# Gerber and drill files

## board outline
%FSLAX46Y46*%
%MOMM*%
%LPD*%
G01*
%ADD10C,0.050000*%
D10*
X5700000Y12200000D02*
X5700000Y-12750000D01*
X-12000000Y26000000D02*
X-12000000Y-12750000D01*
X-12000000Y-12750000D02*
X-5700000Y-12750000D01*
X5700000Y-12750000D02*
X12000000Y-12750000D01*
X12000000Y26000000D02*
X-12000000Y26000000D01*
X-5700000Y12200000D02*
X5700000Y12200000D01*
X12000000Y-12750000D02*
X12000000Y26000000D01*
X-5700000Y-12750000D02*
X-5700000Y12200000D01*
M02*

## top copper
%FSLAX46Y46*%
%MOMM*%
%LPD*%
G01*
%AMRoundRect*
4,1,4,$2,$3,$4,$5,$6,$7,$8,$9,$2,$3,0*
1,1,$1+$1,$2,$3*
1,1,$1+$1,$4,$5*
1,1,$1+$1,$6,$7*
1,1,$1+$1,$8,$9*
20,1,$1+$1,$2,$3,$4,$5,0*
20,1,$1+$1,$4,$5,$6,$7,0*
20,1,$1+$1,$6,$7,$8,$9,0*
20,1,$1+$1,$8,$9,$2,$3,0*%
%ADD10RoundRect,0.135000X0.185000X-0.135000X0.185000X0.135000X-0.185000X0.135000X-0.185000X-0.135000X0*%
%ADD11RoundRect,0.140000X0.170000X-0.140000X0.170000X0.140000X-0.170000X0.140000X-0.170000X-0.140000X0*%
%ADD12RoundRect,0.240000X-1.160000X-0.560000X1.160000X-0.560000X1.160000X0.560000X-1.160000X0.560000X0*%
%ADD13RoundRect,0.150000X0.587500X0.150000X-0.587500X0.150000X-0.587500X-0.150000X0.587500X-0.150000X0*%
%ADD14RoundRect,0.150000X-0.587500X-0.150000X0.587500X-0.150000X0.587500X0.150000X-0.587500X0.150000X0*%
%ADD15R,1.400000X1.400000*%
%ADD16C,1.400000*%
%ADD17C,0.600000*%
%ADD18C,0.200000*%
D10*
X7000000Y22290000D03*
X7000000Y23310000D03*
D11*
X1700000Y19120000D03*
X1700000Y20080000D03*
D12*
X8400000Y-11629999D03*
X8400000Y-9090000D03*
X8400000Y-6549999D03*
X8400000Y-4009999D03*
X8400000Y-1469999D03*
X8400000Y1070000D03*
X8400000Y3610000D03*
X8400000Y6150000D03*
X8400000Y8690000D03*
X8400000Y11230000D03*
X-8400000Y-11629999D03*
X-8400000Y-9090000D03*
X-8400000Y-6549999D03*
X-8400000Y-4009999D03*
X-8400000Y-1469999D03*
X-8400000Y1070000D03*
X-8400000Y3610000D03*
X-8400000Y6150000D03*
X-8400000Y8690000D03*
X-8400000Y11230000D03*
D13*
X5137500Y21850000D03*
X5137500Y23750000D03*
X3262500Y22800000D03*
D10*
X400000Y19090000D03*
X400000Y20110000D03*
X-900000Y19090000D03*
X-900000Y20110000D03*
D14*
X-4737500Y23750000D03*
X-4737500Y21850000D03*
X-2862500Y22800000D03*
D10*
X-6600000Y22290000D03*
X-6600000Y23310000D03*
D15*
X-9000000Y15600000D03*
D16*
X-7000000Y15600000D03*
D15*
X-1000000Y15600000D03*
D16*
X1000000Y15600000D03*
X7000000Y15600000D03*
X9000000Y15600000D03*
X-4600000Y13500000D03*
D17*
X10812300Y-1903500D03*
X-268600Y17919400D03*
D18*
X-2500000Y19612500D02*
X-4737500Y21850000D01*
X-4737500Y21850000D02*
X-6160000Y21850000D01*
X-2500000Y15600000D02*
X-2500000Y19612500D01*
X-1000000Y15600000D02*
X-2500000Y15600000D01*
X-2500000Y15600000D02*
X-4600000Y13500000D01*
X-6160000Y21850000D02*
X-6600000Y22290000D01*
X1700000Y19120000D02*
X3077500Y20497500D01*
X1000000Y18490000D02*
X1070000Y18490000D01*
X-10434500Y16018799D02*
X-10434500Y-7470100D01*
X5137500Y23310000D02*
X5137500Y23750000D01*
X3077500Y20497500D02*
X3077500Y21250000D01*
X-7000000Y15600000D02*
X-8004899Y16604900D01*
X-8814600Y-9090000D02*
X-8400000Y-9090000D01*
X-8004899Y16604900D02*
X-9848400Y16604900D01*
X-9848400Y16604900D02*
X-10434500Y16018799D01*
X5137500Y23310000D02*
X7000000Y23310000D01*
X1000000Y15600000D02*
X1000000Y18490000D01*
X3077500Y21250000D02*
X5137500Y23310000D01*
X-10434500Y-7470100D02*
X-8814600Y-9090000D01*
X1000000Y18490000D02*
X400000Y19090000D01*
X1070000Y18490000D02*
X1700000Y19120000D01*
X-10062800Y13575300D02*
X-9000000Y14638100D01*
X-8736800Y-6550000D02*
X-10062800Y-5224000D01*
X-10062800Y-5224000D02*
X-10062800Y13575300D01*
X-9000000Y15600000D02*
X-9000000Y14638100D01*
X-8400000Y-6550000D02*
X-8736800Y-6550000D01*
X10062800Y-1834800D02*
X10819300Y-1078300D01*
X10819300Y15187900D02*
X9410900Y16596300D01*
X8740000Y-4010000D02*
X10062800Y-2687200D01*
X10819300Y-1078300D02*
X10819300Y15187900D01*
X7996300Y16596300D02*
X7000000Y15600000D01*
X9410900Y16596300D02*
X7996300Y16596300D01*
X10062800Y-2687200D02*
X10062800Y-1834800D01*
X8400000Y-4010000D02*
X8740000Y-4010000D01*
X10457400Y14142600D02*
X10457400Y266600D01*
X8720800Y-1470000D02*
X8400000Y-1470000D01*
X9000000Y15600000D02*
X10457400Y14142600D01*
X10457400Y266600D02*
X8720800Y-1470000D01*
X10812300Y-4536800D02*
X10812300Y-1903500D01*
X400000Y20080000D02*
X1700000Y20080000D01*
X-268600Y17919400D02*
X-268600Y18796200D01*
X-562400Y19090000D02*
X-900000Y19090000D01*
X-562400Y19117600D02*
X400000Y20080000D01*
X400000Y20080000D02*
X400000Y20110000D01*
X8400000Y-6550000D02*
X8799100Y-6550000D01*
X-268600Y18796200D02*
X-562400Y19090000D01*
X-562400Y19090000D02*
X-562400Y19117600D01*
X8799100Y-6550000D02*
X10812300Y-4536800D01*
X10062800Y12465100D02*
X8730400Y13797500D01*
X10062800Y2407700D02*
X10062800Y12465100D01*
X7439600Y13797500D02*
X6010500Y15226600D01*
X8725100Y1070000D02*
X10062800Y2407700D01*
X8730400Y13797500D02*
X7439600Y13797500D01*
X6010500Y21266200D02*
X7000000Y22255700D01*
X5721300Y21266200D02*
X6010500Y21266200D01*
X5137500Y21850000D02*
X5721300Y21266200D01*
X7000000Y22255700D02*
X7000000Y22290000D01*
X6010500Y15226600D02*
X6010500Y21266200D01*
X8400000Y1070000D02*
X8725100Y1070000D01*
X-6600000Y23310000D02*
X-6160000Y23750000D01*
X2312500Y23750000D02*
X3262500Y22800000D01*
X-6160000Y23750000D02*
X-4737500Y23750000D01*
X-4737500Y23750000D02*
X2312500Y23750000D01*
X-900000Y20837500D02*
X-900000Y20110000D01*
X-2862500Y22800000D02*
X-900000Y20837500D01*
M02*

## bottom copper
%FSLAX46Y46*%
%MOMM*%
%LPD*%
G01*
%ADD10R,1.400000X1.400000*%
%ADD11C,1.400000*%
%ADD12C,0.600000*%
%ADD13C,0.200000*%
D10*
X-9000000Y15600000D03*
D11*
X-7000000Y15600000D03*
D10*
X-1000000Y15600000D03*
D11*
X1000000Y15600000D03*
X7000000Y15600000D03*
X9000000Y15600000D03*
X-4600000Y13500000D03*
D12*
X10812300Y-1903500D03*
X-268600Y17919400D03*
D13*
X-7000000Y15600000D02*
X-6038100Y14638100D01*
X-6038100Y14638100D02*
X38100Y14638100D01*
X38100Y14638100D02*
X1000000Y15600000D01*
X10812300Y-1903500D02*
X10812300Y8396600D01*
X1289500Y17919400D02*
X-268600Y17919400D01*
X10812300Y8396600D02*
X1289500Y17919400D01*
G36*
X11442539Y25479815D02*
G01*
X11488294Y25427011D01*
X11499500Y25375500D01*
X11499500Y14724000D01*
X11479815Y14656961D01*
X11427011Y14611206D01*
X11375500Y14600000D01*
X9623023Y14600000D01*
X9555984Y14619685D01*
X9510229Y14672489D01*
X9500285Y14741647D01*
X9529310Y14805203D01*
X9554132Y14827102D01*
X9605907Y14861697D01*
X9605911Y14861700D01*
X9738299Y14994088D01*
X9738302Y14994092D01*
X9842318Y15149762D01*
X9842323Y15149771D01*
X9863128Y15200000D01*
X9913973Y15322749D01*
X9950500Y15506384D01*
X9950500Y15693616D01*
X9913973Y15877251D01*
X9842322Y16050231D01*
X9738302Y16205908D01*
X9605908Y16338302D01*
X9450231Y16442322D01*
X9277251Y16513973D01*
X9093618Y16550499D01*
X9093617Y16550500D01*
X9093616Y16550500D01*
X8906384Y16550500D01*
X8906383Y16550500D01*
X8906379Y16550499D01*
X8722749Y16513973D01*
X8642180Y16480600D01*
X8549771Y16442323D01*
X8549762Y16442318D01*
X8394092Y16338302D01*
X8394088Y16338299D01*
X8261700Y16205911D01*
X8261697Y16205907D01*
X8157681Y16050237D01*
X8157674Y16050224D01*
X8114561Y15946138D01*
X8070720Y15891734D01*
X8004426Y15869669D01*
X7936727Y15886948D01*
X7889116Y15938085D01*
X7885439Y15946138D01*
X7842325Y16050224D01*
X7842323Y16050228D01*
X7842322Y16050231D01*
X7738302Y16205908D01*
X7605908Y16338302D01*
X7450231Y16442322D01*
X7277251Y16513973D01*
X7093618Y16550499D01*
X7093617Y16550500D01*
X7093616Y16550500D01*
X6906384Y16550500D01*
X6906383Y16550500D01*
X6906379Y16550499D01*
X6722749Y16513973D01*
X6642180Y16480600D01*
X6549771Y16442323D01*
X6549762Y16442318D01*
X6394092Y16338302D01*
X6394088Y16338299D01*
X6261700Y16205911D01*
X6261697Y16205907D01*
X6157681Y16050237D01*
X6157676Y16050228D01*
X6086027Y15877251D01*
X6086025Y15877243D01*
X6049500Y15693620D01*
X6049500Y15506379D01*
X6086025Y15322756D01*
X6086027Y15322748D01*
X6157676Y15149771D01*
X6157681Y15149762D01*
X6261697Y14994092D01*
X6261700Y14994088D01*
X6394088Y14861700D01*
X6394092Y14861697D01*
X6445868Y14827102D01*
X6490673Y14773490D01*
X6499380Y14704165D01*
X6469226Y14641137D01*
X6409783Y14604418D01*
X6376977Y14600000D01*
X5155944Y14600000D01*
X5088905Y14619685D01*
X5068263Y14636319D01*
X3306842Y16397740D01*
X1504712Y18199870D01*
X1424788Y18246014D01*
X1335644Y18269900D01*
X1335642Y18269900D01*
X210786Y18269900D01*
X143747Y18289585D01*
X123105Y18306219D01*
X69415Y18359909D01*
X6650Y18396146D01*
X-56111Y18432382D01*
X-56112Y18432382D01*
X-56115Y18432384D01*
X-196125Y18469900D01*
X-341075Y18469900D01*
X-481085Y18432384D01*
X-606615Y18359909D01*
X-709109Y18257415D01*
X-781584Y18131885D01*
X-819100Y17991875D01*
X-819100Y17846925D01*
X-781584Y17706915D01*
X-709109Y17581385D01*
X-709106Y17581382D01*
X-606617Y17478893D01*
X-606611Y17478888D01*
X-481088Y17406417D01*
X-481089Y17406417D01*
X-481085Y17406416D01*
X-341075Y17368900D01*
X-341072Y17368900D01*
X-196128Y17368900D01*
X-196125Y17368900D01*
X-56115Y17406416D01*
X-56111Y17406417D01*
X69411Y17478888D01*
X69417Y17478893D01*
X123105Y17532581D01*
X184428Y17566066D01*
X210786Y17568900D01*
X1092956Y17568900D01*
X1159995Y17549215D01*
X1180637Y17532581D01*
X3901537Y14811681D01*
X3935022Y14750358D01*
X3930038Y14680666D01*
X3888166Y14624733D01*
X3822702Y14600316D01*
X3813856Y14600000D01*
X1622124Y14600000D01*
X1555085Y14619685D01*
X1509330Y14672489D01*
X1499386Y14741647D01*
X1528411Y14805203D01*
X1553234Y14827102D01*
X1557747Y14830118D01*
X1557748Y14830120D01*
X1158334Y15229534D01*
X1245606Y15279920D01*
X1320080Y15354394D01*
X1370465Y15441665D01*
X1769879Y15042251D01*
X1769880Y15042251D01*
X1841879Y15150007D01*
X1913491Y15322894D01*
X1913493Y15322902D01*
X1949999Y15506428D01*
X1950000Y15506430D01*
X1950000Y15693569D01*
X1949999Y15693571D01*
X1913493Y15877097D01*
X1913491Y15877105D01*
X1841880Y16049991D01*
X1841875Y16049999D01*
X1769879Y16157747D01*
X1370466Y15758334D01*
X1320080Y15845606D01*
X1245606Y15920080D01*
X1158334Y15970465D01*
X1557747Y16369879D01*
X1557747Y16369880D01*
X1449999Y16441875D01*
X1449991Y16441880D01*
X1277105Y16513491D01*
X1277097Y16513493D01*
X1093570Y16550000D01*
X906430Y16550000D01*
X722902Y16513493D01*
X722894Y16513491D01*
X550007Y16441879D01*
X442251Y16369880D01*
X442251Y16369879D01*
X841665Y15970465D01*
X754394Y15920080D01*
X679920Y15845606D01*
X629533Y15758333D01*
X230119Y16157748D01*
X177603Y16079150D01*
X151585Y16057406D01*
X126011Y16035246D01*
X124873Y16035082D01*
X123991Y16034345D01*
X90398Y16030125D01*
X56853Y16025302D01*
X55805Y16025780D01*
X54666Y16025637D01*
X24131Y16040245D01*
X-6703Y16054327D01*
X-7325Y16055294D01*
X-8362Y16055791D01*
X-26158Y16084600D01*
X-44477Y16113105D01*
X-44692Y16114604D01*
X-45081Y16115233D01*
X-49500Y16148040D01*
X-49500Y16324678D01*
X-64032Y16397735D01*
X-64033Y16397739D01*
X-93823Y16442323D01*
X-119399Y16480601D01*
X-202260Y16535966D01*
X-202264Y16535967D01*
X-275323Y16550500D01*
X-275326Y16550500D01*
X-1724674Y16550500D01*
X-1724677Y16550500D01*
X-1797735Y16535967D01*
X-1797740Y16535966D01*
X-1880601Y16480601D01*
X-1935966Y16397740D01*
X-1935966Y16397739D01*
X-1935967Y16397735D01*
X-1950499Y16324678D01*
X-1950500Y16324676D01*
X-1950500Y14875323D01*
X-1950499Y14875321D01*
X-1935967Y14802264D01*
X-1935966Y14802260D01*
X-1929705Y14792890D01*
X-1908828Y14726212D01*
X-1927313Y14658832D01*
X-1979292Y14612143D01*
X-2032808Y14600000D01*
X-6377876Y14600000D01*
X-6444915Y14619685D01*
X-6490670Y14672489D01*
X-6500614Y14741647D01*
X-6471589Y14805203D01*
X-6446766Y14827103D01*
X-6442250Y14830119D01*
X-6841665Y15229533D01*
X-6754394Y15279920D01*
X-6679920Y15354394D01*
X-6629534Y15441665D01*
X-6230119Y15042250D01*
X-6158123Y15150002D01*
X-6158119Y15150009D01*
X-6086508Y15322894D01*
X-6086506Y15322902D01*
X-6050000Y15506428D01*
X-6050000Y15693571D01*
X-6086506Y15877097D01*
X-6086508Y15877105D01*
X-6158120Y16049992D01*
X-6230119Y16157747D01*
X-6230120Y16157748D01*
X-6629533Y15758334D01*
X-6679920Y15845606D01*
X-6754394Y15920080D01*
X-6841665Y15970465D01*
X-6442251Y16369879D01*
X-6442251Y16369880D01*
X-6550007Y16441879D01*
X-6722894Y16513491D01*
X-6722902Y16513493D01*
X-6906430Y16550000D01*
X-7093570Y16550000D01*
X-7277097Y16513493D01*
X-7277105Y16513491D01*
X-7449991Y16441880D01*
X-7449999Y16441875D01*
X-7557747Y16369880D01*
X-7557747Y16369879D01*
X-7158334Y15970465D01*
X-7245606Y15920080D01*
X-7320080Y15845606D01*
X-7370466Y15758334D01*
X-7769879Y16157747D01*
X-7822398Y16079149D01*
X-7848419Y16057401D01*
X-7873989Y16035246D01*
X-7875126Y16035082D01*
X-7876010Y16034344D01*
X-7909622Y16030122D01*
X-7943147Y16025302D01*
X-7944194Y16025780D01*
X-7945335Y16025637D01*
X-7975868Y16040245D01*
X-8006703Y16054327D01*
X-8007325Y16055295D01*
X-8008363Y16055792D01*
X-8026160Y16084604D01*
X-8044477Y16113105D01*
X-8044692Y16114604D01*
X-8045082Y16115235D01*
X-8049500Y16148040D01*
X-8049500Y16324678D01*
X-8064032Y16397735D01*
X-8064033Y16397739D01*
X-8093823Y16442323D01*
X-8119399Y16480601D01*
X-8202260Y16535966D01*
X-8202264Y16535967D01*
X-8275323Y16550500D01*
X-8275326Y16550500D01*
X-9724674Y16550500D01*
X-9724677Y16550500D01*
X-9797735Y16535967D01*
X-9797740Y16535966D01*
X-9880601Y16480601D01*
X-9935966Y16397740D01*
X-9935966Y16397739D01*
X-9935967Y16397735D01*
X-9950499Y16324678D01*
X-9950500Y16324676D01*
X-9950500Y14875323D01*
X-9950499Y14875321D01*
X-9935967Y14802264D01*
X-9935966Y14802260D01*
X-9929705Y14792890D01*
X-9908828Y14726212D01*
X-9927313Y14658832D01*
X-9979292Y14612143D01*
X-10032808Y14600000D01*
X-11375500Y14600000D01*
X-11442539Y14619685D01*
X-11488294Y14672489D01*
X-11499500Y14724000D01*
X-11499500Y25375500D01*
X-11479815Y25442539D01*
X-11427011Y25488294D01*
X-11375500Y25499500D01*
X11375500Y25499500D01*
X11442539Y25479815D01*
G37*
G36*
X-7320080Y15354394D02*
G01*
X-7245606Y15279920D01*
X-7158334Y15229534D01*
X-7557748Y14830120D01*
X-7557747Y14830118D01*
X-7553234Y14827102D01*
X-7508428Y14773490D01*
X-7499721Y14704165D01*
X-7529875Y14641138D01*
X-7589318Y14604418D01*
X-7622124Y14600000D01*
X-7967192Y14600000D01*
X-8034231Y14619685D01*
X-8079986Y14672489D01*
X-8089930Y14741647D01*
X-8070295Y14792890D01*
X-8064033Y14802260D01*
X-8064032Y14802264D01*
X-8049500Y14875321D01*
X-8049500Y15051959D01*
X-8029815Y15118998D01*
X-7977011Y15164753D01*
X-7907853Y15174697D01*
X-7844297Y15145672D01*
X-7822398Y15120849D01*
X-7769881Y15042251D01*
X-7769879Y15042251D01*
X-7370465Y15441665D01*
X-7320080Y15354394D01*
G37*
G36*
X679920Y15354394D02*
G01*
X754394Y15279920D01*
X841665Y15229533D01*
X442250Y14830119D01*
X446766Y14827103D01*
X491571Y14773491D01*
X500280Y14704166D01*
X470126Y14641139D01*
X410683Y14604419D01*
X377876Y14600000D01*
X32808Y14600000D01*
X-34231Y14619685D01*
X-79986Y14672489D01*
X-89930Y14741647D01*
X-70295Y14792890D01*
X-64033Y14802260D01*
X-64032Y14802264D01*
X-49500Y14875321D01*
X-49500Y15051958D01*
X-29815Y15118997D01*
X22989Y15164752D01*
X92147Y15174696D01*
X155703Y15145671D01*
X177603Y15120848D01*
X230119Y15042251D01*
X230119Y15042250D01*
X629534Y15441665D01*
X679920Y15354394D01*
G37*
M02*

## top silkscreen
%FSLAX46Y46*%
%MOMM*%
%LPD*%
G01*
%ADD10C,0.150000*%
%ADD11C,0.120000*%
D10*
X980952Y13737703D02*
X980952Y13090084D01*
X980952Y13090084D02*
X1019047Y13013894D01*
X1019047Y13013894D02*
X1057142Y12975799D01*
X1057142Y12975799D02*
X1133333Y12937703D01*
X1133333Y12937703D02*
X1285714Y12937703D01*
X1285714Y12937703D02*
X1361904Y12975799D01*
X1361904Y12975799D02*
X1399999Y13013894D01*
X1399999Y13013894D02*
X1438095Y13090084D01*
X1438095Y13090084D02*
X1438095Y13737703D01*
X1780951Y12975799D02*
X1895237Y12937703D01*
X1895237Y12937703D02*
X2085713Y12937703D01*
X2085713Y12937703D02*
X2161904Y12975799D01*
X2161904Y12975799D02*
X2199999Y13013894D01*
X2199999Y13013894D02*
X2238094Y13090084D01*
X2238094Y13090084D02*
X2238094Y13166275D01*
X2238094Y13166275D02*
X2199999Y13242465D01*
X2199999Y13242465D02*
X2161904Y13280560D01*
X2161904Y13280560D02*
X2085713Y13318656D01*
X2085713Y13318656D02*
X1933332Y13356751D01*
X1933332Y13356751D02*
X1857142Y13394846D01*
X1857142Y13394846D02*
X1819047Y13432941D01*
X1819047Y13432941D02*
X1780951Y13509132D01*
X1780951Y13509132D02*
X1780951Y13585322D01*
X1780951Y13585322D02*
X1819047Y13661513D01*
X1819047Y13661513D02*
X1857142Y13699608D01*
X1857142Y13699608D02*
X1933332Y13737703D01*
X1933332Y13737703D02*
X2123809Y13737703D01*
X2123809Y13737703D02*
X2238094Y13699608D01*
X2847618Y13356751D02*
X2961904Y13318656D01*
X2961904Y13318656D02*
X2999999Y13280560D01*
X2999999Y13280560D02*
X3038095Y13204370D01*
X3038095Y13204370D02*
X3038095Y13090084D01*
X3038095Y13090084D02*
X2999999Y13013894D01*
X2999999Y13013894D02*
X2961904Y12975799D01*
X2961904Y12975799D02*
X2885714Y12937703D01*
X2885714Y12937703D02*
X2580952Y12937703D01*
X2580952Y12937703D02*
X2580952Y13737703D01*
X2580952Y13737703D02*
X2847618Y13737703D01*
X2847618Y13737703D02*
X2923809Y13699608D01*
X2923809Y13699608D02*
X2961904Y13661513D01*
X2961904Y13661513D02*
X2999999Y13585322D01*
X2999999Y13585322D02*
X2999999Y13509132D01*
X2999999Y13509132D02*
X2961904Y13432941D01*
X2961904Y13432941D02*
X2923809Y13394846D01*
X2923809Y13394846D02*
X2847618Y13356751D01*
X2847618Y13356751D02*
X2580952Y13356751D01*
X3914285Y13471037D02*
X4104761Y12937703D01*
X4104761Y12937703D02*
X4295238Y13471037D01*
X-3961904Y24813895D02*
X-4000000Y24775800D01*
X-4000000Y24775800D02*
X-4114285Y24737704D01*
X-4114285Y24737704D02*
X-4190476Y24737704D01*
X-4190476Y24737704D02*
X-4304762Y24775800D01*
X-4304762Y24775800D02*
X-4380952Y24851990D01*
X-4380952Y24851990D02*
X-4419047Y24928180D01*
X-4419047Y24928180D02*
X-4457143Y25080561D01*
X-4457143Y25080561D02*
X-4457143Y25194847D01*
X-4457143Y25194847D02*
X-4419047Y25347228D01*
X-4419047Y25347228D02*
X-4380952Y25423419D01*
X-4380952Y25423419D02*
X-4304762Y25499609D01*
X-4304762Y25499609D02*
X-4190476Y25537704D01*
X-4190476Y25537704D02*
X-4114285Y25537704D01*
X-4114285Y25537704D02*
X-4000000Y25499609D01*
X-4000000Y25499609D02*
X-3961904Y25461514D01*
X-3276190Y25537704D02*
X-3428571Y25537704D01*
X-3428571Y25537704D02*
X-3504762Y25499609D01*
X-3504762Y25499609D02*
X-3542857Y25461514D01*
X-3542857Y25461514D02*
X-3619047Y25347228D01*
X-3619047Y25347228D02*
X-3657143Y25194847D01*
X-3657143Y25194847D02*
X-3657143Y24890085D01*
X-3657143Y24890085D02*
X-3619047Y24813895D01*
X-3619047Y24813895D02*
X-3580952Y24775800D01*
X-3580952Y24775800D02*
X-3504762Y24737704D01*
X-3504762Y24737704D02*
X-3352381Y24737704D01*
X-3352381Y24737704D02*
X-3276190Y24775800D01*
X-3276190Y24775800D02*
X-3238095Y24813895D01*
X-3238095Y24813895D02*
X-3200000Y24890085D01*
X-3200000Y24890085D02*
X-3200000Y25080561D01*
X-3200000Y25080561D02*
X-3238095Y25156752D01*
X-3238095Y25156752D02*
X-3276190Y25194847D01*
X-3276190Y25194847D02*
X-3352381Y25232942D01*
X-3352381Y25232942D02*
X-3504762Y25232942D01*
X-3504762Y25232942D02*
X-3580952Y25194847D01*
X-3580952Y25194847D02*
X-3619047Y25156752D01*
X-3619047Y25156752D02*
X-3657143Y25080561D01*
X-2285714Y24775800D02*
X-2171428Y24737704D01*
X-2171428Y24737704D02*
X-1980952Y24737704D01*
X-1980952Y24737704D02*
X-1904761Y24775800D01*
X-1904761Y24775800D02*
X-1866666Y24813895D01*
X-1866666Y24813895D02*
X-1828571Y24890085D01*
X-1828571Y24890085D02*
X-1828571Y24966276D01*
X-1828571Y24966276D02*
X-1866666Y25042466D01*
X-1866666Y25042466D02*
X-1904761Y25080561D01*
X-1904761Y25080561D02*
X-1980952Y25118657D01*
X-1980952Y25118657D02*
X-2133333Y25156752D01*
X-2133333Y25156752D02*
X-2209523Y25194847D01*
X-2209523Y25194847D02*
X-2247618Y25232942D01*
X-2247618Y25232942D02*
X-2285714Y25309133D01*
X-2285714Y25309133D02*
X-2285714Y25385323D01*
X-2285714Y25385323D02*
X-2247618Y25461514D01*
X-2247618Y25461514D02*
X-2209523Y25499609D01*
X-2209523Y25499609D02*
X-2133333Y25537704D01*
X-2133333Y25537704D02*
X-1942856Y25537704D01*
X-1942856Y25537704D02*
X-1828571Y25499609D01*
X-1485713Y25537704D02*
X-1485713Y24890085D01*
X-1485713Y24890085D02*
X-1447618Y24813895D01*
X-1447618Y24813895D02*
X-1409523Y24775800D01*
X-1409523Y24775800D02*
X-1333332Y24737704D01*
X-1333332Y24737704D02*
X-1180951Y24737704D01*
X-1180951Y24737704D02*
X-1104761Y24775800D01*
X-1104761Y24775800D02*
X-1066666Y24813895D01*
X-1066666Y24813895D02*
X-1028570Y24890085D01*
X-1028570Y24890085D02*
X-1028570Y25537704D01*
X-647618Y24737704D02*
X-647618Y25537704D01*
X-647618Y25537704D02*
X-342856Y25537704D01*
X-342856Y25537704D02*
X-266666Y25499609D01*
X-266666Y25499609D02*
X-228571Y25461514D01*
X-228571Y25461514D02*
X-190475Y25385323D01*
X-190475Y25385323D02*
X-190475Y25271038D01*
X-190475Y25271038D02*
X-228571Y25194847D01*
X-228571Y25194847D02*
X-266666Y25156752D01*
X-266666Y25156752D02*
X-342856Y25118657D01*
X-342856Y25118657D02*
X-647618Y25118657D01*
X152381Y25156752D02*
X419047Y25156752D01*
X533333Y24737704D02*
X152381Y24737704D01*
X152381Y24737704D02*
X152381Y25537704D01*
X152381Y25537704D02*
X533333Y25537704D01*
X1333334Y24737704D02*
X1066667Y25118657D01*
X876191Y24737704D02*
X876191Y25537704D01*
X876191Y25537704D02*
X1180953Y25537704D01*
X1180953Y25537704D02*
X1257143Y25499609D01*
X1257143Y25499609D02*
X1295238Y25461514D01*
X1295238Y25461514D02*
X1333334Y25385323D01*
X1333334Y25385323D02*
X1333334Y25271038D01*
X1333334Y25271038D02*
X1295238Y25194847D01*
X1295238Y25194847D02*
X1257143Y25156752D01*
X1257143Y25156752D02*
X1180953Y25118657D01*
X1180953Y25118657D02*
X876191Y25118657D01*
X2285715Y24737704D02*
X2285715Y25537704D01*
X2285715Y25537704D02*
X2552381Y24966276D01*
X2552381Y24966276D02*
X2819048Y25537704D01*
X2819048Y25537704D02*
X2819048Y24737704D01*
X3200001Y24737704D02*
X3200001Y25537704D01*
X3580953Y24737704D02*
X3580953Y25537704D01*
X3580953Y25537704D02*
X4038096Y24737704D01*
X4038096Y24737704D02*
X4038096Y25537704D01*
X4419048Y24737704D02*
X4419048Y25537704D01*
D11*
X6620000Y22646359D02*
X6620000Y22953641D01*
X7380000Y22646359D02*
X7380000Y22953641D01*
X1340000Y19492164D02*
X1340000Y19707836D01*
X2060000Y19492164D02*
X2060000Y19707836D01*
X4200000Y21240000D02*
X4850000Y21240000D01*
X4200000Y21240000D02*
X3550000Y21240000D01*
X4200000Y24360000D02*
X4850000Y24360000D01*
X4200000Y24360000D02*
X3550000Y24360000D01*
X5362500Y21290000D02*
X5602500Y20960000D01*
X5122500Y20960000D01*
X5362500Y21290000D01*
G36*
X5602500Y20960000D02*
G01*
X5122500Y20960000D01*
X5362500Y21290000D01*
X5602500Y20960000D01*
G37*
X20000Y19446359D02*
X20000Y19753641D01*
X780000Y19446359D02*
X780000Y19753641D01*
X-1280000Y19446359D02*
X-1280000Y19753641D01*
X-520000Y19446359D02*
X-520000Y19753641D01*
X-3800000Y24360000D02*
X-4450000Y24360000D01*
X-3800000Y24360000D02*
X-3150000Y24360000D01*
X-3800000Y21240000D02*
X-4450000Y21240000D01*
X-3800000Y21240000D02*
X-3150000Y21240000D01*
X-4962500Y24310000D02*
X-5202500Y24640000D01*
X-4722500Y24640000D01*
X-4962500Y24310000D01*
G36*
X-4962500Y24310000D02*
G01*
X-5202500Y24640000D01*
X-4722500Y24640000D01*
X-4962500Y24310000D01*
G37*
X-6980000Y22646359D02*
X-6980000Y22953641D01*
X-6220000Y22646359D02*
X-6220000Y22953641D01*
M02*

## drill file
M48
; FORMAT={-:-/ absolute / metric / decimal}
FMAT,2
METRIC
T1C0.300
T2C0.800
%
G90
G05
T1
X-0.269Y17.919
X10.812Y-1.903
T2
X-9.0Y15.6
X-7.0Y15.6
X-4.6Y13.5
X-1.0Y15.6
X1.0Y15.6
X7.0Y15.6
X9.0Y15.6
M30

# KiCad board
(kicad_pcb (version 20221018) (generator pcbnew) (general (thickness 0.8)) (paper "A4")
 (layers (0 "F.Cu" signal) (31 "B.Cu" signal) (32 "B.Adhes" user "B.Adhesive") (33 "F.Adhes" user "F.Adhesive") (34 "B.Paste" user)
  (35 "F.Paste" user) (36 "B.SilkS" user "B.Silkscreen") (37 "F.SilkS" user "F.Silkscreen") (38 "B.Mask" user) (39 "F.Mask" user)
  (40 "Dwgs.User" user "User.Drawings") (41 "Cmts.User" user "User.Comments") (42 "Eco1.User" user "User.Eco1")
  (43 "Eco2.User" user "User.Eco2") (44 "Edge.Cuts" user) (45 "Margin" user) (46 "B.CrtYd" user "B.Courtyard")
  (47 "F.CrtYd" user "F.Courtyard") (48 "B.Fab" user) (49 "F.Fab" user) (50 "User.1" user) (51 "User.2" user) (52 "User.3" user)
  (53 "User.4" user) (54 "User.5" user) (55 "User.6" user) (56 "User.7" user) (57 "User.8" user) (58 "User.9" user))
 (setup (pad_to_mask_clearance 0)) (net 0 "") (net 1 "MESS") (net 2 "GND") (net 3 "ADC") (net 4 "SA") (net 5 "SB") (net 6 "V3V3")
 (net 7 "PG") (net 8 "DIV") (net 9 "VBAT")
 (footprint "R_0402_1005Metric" (layer "F.Cu") (at 7 -22.8 90)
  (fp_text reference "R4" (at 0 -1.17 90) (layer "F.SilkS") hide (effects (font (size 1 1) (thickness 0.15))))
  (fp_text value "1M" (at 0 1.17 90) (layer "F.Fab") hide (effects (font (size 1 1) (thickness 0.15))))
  (fp_line (start -0.153641 -0.38) (end 0.153641 -0.38) (stroke (width 0.12) (type solid)) (layer "F.SilkS"))
  (fp_line (start -0.153641 0.38) (end 0.153641 0.38) (stroke (width 0.12) (type solid)) (layer "F.SilkS"))
  (pad "1" smd roundrect (at -0.51 0 90) (size 0.54 0.64) (layers "F.Cu" "F.Paste" "F.Mask") (roundrect_rratio 0.25) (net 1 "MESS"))
  (pad "2" smd roundrect (at 0.51 0 90) (size 0.54 0.64) (layers "F.Cu" "F.Paste" "F.Mask") (roundrect_rratio 0.25) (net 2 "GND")))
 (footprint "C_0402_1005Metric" (layer "F.Cu") (at 1.7 -19.6 90)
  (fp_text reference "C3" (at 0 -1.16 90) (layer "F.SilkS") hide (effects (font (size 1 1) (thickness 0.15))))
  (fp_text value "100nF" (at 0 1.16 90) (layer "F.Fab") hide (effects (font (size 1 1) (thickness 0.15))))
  (fp_line (start -0.107836 -0.36) (end 0.107836 -0.36) (stroke (width 0.12) (type solid)) (layer "F.SilkS"))
  (fp_line (start -0.107836 0.36) (end 0.107836 0.36) (stroke (width 0.12) (type solid)) (layer "F.SilkS"))
  (pad "1" smd roundrect (at -0.48 0 90) (size 0.56 0.62) (layers "F.Cu" "F.Paste" "F.Mask") (roundrect_rratio 0.25) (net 2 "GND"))
  (pad "2" smd roundrect (at 0.48 0 90) (size 0.56 0.62) (layers "F.Cu" "F.Paste" "F.Mask") (roundrect_rratio 0.25) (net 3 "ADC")))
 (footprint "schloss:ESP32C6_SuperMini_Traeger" (layer "F.Cu") (at 0 0)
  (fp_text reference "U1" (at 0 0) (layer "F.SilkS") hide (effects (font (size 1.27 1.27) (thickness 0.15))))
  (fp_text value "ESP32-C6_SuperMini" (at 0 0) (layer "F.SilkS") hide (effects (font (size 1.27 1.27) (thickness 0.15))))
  (pad "1" smd roundrect (at 8.4 11.629999) (size 2.8 1.6) (layers "F.Cu" "F.Mask") (roundrect_rratio 0.15) (thermal_bridge_angle 45))
  (pad "2" smd roundrect (at 8.4 9.09) (size 2.8 1.6) (layers "F.Cu" "F.Mask") (roundrect_rratio 0.15) (thermal_bridge_angle 45))
  (pad "3" smd roundrect (at 8.4 6.549999) (size 2.8 1.6) (layers "F.Cu" "F.Mask") (roundrect_rratio 0.15) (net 3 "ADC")
   (thermal_bridge_angle 45))
  (pad "4" smd roundrect (at 8.4 4.009999) (size 2.8 1.6) (layers "F.Cu" "F.Mask") (roundrect_rratio 0.15) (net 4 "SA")
   (thermal_bridge_angle 45))
  (pad "5" smd roundrect (at 8.4 1.469999) (size 2.8 1.6) (layers "F.Cu" "F.Mask") (roundrect_rratio 0.15) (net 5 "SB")
   (thermal_bridge_angle 45))
  (pad "6" smd roundrect (at 8.4 -1.07) (size 2.8 1.6) (layers "F.Cu" "F.Mask") (roundrect_rratio 0.15) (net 1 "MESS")
   (thermal_bridge_angle 45))
  (pad "7" smd roundrect (at 8.4 -3.61) (size 2.8 1.6) (layers "F.Cu" "F.Mask") (roundrect_rratio 0.15) (thermal_bridge_angle 45))
  (pad "8" smd roundrect (at 8.4 -6.15) (size 2.8 1.6) (layers "F.Cu" "F.Mask") (roundrect_rratio 0.15) (thermal_bridge_angle 45))
  (pad "9" smd roundrect (at 8.4 -8.69) (size 2.8 1.6) (layers "F.Cu" "F.Mask") (roundrect_rratio 0.15) (thermal_bridge_angle 45))
  (pad "10" smd roundrect (at 8.4 -11.23) (size 2.8 1.6) (layers "F.Cu" "F.Mask") (roundrect_rratio 0.15) (thermal_bridge_angle 45))
  (pad "11" smd roundrect (at -8.4 11.629999) (size 2.8 1.6) (layers "F.Cu" "F.Mask") (roundrect_rratio 0.15) (thermal_bridge_angle 45))
  (pad "12" smd roundrect (at -8.4 9.09) (size 2.8 1.6) (layers "F.Cu" "F.Mask") (roundrect_rratio 0.15) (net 2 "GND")
   (thermal_bridge_angle 45))
  (pad "13" smd roundrect (at -8.4 6.549999) (size 2.8 1.6) (layers "F.Cu" "F.Mask") (roundrect_rratio 0.15) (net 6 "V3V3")
   (thermal_bridge_angle 45))
  (pad "14" smd roundrect (at -8.4 4.009999) (size 2.8 1.6) (layers "F.Cu" "F.Mask") (roundrect_rratio 0.15) (thermal_bridge_angle 45))
  (pad "15" smd roundrect (at -8.4 1.469999) (size 2.8 1.6) (layers "F.Cu" "F.Mask") (roundrect_rratio 0.15) (thermal_bridge_angle 45))
  (pad "16" smd roundrect (at -8.4 -1.07) (size 2.8 1.6) (layers "F.Cu" "F.Mask") (roundrect_rratio 0.15) (thermal_bridge_angle 45))
  (pad "17" smd roundrect (at -8.4 -3.61) (size 2.8 1.6) (layers "F.Cu" "F.Mask") (roundrect_rratio 0.15) (thermal_bridge_angle 45))
  (pad "18" smd roundrect (at -8.4 -6.15) (size 2.8 1.6) (layers "F.Cu" "F.Mask") (roundrect_rratio 0.15) (thermal_bridge_angle 45))
  (pad "19" smd roundrect (at -8.4 -8.69) (size 2.8 1.6) (layers "F.Cu" "F.Mask") (roundrect_rratio 0.15) (thermal_bridge_angle 45))
  (pad "20" smd roundrect (at -8.4 -11.23) (size 2.8 1.6) (layers "F.Cu" "F.Mask") (roundrect_rratio 0.15) (thermal_bridge_angle 45)))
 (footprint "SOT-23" (layer "F.Cu") (at 4.2 -22.8 180)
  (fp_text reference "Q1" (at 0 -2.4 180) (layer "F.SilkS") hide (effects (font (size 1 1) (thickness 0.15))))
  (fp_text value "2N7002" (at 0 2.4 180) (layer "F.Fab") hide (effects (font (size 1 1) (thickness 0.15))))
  (fp_line (start 0 -1.56) (end -0.65 -1.56) (stroke (width 0.12) (type solid)) (layer "F.SilkS"))
  (fp_line (start 0 -1.56) (end 0.65 -1.56) (stroke (width 0.12) (type solid)) (layer "F.SilkS"))
  (fp_line (start 0 1.56) (end -0.65 1.56) (stroke (width 0.12) (type solid)) (layer "F.SilkS"))
  (fp_line (start 0 1.56) (end 0.65 1.56) (stroke (width 0.12) (type solid)) (layer "F.SilkS"))
  (fp_poly
   (pts (xy -1.1625 -1.51) (xy -1.4025 -1.84) (xy -0.9225 -1.84) (xy -1.1625 -1.51)) (stroke (width 0.12) (type solid)) (fill solid)
   (layer "F.SilkS"))
  (pad "1" smd roundrect (at -0.9375 -0.95 180) (size 1.475 0.6) (layers "F.Cu" "F.Paste" "F.Mask") (roundrect_rratio 0.25) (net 1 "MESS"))
  (pad "2" smd roundrect (at -0.9375 0.95 180) (size 1.475 0.6) (layers "F.Cu" "F.Paste" "F.Mask") (roundrect_rratio 0.25) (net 2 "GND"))
  (pad "3" smd roundrect (at 0.9375 0 180) (size 1.475 0.6) (layers "F.Cu" "F.Paste" "F.Mask") (roundrect_rratio 0.25) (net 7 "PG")))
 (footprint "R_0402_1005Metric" (layer "F.Cu") (at 0.4 -19.6 90)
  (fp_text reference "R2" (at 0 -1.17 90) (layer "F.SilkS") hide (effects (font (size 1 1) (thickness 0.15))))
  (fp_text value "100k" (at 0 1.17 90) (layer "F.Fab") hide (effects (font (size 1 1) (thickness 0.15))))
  (fp_line (start -0.153641 -0.38) (end 0.153641 -0.38) (stroke (width 0.12) (type solid)) (layer "F.SilkS"))
  (fp_line (start -0.153641 0.38) (end 0.153641 0.38) (stroke (width 0.12) (type solid)) (layer "F.SilkS"))
  (pad "1" smd roundrect (at -0.51 0 90) (size 0.54 0.64) (layers "F.Cu" "F.Paste" "F.Mask") (roundrect_rratio 0.25) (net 2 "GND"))
  (pad "2" smd roundrect (at 0.51 0 90) (size 0.54 0.64) (layers "F.Cu" "F.Paste" "F.Mask") (roundrect_rratio 0.25) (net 3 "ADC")))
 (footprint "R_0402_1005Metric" (layer "F.Cu") (at -0.9 -19.6 90)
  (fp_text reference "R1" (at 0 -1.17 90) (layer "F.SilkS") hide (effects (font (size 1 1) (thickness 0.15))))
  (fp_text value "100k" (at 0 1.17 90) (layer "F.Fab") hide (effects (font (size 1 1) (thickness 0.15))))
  (fp_line (start -0.153641 -0.38) (end 0.153641 -0.38) (stroke (width 0.12) (type solid)) (layer "F.SilkS"))
  (fp_line (start -0.153641 0.38) (end 0.153641 0.38) (stroke (width 0.12) (type solid)) (layer "F.SilkS"))
  (pad "1" smd roundrect (at -0.51 0 90) (size 0.54 0.64) (layers "F.Cu" "F.Paste" "F.Mask") (roundrect_rratio 0.25) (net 3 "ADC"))
  (pad "2" smd roundrect (at 0.51 0 90) (size 0.54 0.64) (layers "F.Cu" "F.Paste" "F.Mask") (roundrect_rratio 0.25) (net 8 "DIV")))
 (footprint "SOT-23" (layer "F.Cu") (at -3.8 -22.8)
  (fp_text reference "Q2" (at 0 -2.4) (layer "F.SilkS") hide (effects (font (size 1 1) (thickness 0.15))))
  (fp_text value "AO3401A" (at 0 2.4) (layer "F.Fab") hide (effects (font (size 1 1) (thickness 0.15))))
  (fp_line (start 0 -1.56) (end -0.65 -1.56) (stroke (width 0.12) (type solid)) (layer "F.SilkS"))
  (fp_line (start 0 -1.56) (end 0.65 -1.56) (stroke (width 0.12) (type solid)) (layer "F.SilkS"))
  (fp_line (start 0 1.56) (end -0.65 1.56) (stroke (width 0.12) (type solid)) (layer "F.SilkS"))
  (fp_line (start 0 1.56) (end 0.65 1.56) (stroke (width 0.12) (type solid)) (layer "F.SilkS"))
  (fp_poly
   (pts (xy -1.1625 -1.51) (xy -1.4025 -1.84) (xy -0.9225 -1.84) (xy -1.1625 -1.51)) (stroke (width 0.12) (type solid)) (fill solid)
   (layer "F.SilkS"))
  (pad "1" smd roundrect (at -0.9375 -0.95) (size 1.475 0.6) (layers "F.Cu" "F.Paste" "F.Mask") (roundrect_rratio 0.25) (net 7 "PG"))
  (pad "2" smd roundrect (at -0.9375 0.95) (size 1.475 0.6) (layers "F.Cu" "F.Paste" "F.Mask") (roundrect_rratio 0.25) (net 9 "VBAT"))
  (pad "3" smd roundrect (at 0.9375 0) (size 1.475 0.6) (layers "F.Cu" "F.Paste" "F.Mask") (roundrect_rratio 0.25) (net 8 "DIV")))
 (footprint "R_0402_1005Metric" (layer "F.Cu") (at -6.6 -22.8 90)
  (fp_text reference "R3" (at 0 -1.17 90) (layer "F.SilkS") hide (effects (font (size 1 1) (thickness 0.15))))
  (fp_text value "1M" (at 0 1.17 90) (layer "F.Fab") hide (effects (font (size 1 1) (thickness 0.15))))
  (fp_line (start -0.153641 -0.38) (end 0.153641 -0.38) (stroke (width 0.12) (type solid)) (layer "F.SilkS"))
  (fp_line (start -0.153641 0.38) (end 0.153641 0.38) (stroke (width 0.12) (type solid)) (layer "F.SilkS"))
  (pad "1" smd roundrect (at -0.51 0 90) (size 0.54 0.64) (layers "F.Cu" "F.Paste" "F.Mask") (roundrect_rratio 0.25) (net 9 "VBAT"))
  (pad "2" smd roundrect (at 0.51 0 90) (size 0.54 0.64) (layers "F.Cu" "F.Paste" "F.Mask") (roundrect_rratio 0.25) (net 7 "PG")))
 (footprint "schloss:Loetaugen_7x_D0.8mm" (layer "F.Cu") (at 0 0)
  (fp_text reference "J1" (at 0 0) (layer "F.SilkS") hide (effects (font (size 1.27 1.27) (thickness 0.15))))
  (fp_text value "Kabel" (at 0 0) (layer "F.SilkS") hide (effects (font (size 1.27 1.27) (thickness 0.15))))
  (pad "1" thru_hole rect (at -9 -15.6) (size 1.4 1.4) (drill 0.8) (layers "*.Cu" "*.Mask") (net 6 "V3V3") (thermal_bridge_angle 45))
  (pad "2" thru_hole circle (at -7 -15.6) (size 1.4 1.4) (drill 0.8) (layers "*.Cu" "*.Mask") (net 2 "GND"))
  (pad "3" thru_hole rect (at -1 -15.6) (size 1.4 1.4) (drill 0.8) (layers "*.Cu" "*.Mask") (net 9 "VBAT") (thermal_bridge_angle 45))
  (pad "4" thru_hole circle (at 1 -15.6) (size 1.4 1.4) (drill 0.8) (layers "*.Cu" "*.Mask") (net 2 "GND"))
  (pad "5" thru_hole circle (at 7 -15.6) (size 1.4 1.4) (drill 0.8) (layers "*.Cu" "*.Mask") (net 4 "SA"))
  (pad "6" thru_hole circle (at 9 -15.6) (size 1.4 1.4) (drill 0.8) (layers "*.Cu" "*.Mask") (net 5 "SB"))
  (pad "7" thru_hole circle (at -4.6 -13.5) (size 1.4 1.4) (drill 0.8) (layers "*.Cu" "*.Mask") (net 9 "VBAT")))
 (gr_line (start 5.7 -12.2) (end 5.7 12.75) (stroke (width 0.05) (type default)) (layer "Edge.Cuts"))
 (gr_line (start -12 -26) (end -12 12.75) (stroke (width 0.05) (type default)) (layer "Edge.Cuts"))
 (gr_line (start -12 12.75) (end -5.7 12.75) (stroke (width 0.05) (type default)) (layer "Edge.Cuts"))
 (gr_line (start 5.7 12.75) (end 12 12.75) (stroke (width 0.05) (type default)) (layer "Edge.Cuts"))
 (gr_line (start 12 -26) (end -12 -26) (stroke (width 0.05) (type default)) (layer "Edge.Cuts"))
 (gr_line (start -5.7 -12.2) (end 5.7 -12.2) (stroke (width 0.05) (type default)) (layer "Edge.Cuts"))
 (gr_line (start 12 12.75) (end 12 -26) (stroke (width 0.05) (type default)) (layer "Edge.Cuts"))
 (gr_line (start -5.7 12.75) (end -5.7 -12.2) (stroke (width 0.05) (type default)) (layer "Edge.Cuts"))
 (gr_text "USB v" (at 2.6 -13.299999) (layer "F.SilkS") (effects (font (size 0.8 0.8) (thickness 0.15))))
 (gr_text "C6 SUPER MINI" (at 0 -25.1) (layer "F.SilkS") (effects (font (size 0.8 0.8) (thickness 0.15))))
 (segment (start -2.5 -19.6125) (end -4.7375 -21.85) (width 0.2) (layer "F.Cu") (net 9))
 (segment (start -4.7375 -21.85) (end -6.16 -21.85) (width 0.2) (layer "F.Cu") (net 9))
 (segment (start -2.5 -15.6) (end -2.5 -19.6125) (width 0.2) (layer "F.Cu") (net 9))
 (segment (start -1 -15.6) (end -2.5 -15.6) (width 0.2) (layer "F.Cu") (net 9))
 (segment (start -2.5 -15.6) (end -4.6 -13.5) (width 0.2) (layer "F.Cu") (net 9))
 (segment (start -6.16 -21.85) (end -6.6 -22.29) (width 0.2) (layer "F.Cu") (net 9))
 (segment (start 1.7 -19.12) (end 3.0775 -20.4975) (width 0.2) (layer "F.Cu") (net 2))
 (segment (start 1 -18.49) (end 1.07 -18.49) (width 0.2) (layer "F.Cu") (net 2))
 (segment (start -10.4345 -16.018799) (end -10.4345 7.4701) (width 0.2) (layer "F.Cu") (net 2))
 (segment (start 5.1375 -23.31) (end 5.1375 -23.75) (width 0.2) (layer "F.Cu") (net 2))
 (segment (start 3.0775 -20.4975) (end 3.0775 -21.25) (width 0.2) (layer "F.Cu") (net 2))
 (segment (start -7 -15.6) (end -8.004899 -16.6049) (width 0.2) (layer "F.Cu") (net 2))
 (segment (start -8.8146 9.09) (end -8.4 9.09) (width 0.2) (layer "F.Cu") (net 2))
 (segment (start -8.004899 -16.6049) (end -9.8484 -16.6049) (width 0.2) (layer "F.Cu") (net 2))
 (segment (start -9.8484 -16.6049) (end -10.4345 -16.018799) (width 0.2) (layer "F.Cu") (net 2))
 (segment (start 5.1375 -23.31) (end 7 -23.31) (width 0.2) (layer "F.Cu") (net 2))
 (segment (start 1 -15.6) (end 1 -18.49) (width 0.2) (layer "F.Cu") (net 2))
 (segment (start 3.0775 -21.25) (end 5.1375 -23.31) (width 0.2) (layer "F.Cu") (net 2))
 (segment (start -10.4345 7.4701) (end -8.8146 9.09) (width 0.2) (layer "F.Cu") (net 2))
 (segment (start 1 -18.49) (end 0.4 -19.09) (width 0.2) (layer "F.Cu") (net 2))
 (segment (start 1.07 -18.49) (end 1.7 -19.12) (width 0.2) (layer "F.Cu") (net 2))
 (segment (start -7 -15.6) (end -6.0381 -14.6381) (width 0.2) (layer "B.Cu") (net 2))
 (segment (start -6.0381 -14.6381) (end 0.0381 -14.6381) (width 0.2) (layer "B.Cu") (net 2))
 (segment (start 0.0381 -14.6381) (end 1 -15.6) (width 0.2) (layer "B.Cu") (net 2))
 (segment (start -10.0628 -13.5753) (end -9 -14.6381) (width 0.2) (layer "F.Cu") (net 6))
 (segment (start -8.7368 6.55) (end -10.0628 5.224) (width 0.2) (layer "F.Cu") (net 6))
 (segment (start -10.0628 5.224) (end -10.0628 -13.5753) (width 0.2) (layer "F.Cu") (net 6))
 (segment (start -9 -15.6) (end -9 -14.6381) (width 0.2) (layer "F.Cu") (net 6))
 (segment (start -8.4 6.55) (end -8.7368 6.55) (width 0.2) (layer "F.Cu") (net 6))
 (segment (start 10.0628 1.8348) (end 10.8193 1.0783) (width 0.2) (layer "F.Cu") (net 4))
 (segment (start 10.8193 -15.1879) (end 9.4109 -16.5963) (width 0.2) (layer "F.Cu") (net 4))
 (segment (start 8.74 4.01) (end 10.0628 2.6872) (width 0.2) (layer "F.Cu") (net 4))
 (segment (start 10.8193 1.0783) (end 10.8193 -15.1879) (width 0.2) (layer "F.Cu") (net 4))
 (segment (start 7.9963 -16.5963) (end 7 -15.6) (width 0.2) (layer "F.Cu") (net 4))
 (segment (start 9.4109 -16.5963) (end 7.9963 -16.5963) (width 0.2) (layer "F.Cu") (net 4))
 (segment (start 10.0628 2.6872) (end 10.0628 1.8348) (width 0.2) (layer "F.Cu") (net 4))
 (segment (start 8.4 4.01) (end 8.74 4.01) (width 0.2) (layer "F.Cu") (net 4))
 (segment (start 10.4574 -14.1426) (end 10.4574 -0.2666) (width 0.2) (layer "F.Cu") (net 5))
 (segment (start 8.7208 1.47) (end 8.4 1.47) (width 0.2) (layer "F.Cu") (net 5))
 (segment (start 9 -15.6) (end 10.4574 -14.1426) (width 0.2) (layer "F.Cu") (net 5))
 (segment (start 10.4574 -0.2666) (end 8.7208 1.47) (width 0.2) (layer "F.Cu") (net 5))
 (segment (start 10.8123 4.5368) (end 10.8123 1.9035) (width 0.2) (layer "F.Cu") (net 3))
 (segment (start 0.4 -20.08) (end 1.7 -20.08) (width 0.2) (layer "F.Cu") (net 3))
 (segment (start -0.2686 -17.9194) (end -0.2686 -18.7962) (width 0.2) (layer "F.Cu") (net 3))
 (segment (start -0.5624 -19.09) (end -0.9 -19.09) (width 0.2) (layer "F.Cu") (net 3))
 (segment (start -0.5624 -19.1176) (end 0.4 -20.08) (width 0.2) (layer "F.Cu") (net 3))
 (segment (start 0.4 -20.08) (end 0.4 -20.11) (width 0.2) (layer "F.Cu") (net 3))
 (segment (start 8.4 6.55) (end 8.7991 6.55) (width 0.2) (layer "F.Cu") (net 3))
 (segment (start -0.2686 -18.7962) (end -0.5624 -19.09) (width 0.2) (layer "F.Cu") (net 3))
 (segment (start -0.5624 -19.09) (end -0.5624 -19.1176) (width 0.2) (layer "F.Cu") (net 3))
 (segment (start 8.7991 6.55) (end 10.8123 4.5368) (width 0.2) (layer "F.Cu") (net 3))
 (via (at 10.8123 1.9035) (size 0.6) (drill 0.3) (layers "F.Cu" "B.Cu") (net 3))
 (via (at -0.2686 -17.9194) (size 0.6) (drill 0.3) (layers "F.Cu" "B.Cu") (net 3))
 (segment (start 10.8123 1.9035) (end 10.8123 -8.3966) (width 0.2) (layer "B.Cu") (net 3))
 (segment (start 1.2895 -17.9194) (end -0.2686 -17.9194) (width 0.2) (layer "B.Cu") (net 3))
 (segment (start 10.8123 -8.3966) (end 1.2895 -17.9194) (width 0.2) (layer "B.Cu") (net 3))
 (segment (start 10.0628 -12.4651) (end 8.7304 -13.7975) (width 0.2) (layer "F.Cu") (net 1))
 (segment (start 10.0628 -2.4077) (end 10.0628 -12.4651) (width 0.2) (layer "F.Cu") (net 1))
 (segment (start 7.4396 -13.7975) (end 6.0105 -15.2266) (width 0.2) (layer "F.Cu") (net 1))
 (segment (start 8.7251 -1.07) (end 10.0628 -2.4077) (width 0.2) (layer "F.Cu") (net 1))
 (segment (start 8.7304 -13.7975) (end 7.4396 -13.7975) (width 0.2) (layer "F.Cu") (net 1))
 (segment (start 6.0105 -21.2662) (end 7 -22.2557) (width 0.2) (layer "F.Cu") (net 1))
 (segment (start 5.7213 -21.2662) (end 6.0105 -21.2662) (width 0.2) (layer "F.Cu") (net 1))
 (segment (start 5.1375 -21.85) (end 5.7213 -21.2662) (width 0.2) (layer "F.Cu") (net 1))
 (segment (start 7 -22.2557) (end 7 -22.29) (width 0.2) (layer "F.Cu") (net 1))
 (segment (start 6.0105 -15.2266) (end 6.0105 -21.2662) (width 0.2) (layer "F.Cu") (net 1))
 (segment (start 8.4 -1.07) (end 8.7251 -1.07) (width 0.2) (layer "F.Cu") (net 1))
 (segment (start -6.6 -23.31) (end -6.16 -23.75) (width 0.2) (layer "F.Cu") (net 7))
 (segment (start 2.3125 -23.75) (end 3.2625 -22.8) (width 0.2) (layer "F.Cu") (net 7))
 (segment (start -6.16 -23.75) (end -4.7375 -23.75) (width 0.2) (layer "F.Cu") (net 7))
 (segment (start -4.7375 -23.75) (end 2.3125 -23.75) (width 0.2) (layer "F.Cu") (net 7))
 (segment (start -0.9 -20.8375) (end -0.9 -20.11) (width 0.2) (layer "F.Cu") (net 8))
 (segment (start -2.8625 -22.8) (end -0.9 -20.8375) (width 0.2) (layer "F.Cu") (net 8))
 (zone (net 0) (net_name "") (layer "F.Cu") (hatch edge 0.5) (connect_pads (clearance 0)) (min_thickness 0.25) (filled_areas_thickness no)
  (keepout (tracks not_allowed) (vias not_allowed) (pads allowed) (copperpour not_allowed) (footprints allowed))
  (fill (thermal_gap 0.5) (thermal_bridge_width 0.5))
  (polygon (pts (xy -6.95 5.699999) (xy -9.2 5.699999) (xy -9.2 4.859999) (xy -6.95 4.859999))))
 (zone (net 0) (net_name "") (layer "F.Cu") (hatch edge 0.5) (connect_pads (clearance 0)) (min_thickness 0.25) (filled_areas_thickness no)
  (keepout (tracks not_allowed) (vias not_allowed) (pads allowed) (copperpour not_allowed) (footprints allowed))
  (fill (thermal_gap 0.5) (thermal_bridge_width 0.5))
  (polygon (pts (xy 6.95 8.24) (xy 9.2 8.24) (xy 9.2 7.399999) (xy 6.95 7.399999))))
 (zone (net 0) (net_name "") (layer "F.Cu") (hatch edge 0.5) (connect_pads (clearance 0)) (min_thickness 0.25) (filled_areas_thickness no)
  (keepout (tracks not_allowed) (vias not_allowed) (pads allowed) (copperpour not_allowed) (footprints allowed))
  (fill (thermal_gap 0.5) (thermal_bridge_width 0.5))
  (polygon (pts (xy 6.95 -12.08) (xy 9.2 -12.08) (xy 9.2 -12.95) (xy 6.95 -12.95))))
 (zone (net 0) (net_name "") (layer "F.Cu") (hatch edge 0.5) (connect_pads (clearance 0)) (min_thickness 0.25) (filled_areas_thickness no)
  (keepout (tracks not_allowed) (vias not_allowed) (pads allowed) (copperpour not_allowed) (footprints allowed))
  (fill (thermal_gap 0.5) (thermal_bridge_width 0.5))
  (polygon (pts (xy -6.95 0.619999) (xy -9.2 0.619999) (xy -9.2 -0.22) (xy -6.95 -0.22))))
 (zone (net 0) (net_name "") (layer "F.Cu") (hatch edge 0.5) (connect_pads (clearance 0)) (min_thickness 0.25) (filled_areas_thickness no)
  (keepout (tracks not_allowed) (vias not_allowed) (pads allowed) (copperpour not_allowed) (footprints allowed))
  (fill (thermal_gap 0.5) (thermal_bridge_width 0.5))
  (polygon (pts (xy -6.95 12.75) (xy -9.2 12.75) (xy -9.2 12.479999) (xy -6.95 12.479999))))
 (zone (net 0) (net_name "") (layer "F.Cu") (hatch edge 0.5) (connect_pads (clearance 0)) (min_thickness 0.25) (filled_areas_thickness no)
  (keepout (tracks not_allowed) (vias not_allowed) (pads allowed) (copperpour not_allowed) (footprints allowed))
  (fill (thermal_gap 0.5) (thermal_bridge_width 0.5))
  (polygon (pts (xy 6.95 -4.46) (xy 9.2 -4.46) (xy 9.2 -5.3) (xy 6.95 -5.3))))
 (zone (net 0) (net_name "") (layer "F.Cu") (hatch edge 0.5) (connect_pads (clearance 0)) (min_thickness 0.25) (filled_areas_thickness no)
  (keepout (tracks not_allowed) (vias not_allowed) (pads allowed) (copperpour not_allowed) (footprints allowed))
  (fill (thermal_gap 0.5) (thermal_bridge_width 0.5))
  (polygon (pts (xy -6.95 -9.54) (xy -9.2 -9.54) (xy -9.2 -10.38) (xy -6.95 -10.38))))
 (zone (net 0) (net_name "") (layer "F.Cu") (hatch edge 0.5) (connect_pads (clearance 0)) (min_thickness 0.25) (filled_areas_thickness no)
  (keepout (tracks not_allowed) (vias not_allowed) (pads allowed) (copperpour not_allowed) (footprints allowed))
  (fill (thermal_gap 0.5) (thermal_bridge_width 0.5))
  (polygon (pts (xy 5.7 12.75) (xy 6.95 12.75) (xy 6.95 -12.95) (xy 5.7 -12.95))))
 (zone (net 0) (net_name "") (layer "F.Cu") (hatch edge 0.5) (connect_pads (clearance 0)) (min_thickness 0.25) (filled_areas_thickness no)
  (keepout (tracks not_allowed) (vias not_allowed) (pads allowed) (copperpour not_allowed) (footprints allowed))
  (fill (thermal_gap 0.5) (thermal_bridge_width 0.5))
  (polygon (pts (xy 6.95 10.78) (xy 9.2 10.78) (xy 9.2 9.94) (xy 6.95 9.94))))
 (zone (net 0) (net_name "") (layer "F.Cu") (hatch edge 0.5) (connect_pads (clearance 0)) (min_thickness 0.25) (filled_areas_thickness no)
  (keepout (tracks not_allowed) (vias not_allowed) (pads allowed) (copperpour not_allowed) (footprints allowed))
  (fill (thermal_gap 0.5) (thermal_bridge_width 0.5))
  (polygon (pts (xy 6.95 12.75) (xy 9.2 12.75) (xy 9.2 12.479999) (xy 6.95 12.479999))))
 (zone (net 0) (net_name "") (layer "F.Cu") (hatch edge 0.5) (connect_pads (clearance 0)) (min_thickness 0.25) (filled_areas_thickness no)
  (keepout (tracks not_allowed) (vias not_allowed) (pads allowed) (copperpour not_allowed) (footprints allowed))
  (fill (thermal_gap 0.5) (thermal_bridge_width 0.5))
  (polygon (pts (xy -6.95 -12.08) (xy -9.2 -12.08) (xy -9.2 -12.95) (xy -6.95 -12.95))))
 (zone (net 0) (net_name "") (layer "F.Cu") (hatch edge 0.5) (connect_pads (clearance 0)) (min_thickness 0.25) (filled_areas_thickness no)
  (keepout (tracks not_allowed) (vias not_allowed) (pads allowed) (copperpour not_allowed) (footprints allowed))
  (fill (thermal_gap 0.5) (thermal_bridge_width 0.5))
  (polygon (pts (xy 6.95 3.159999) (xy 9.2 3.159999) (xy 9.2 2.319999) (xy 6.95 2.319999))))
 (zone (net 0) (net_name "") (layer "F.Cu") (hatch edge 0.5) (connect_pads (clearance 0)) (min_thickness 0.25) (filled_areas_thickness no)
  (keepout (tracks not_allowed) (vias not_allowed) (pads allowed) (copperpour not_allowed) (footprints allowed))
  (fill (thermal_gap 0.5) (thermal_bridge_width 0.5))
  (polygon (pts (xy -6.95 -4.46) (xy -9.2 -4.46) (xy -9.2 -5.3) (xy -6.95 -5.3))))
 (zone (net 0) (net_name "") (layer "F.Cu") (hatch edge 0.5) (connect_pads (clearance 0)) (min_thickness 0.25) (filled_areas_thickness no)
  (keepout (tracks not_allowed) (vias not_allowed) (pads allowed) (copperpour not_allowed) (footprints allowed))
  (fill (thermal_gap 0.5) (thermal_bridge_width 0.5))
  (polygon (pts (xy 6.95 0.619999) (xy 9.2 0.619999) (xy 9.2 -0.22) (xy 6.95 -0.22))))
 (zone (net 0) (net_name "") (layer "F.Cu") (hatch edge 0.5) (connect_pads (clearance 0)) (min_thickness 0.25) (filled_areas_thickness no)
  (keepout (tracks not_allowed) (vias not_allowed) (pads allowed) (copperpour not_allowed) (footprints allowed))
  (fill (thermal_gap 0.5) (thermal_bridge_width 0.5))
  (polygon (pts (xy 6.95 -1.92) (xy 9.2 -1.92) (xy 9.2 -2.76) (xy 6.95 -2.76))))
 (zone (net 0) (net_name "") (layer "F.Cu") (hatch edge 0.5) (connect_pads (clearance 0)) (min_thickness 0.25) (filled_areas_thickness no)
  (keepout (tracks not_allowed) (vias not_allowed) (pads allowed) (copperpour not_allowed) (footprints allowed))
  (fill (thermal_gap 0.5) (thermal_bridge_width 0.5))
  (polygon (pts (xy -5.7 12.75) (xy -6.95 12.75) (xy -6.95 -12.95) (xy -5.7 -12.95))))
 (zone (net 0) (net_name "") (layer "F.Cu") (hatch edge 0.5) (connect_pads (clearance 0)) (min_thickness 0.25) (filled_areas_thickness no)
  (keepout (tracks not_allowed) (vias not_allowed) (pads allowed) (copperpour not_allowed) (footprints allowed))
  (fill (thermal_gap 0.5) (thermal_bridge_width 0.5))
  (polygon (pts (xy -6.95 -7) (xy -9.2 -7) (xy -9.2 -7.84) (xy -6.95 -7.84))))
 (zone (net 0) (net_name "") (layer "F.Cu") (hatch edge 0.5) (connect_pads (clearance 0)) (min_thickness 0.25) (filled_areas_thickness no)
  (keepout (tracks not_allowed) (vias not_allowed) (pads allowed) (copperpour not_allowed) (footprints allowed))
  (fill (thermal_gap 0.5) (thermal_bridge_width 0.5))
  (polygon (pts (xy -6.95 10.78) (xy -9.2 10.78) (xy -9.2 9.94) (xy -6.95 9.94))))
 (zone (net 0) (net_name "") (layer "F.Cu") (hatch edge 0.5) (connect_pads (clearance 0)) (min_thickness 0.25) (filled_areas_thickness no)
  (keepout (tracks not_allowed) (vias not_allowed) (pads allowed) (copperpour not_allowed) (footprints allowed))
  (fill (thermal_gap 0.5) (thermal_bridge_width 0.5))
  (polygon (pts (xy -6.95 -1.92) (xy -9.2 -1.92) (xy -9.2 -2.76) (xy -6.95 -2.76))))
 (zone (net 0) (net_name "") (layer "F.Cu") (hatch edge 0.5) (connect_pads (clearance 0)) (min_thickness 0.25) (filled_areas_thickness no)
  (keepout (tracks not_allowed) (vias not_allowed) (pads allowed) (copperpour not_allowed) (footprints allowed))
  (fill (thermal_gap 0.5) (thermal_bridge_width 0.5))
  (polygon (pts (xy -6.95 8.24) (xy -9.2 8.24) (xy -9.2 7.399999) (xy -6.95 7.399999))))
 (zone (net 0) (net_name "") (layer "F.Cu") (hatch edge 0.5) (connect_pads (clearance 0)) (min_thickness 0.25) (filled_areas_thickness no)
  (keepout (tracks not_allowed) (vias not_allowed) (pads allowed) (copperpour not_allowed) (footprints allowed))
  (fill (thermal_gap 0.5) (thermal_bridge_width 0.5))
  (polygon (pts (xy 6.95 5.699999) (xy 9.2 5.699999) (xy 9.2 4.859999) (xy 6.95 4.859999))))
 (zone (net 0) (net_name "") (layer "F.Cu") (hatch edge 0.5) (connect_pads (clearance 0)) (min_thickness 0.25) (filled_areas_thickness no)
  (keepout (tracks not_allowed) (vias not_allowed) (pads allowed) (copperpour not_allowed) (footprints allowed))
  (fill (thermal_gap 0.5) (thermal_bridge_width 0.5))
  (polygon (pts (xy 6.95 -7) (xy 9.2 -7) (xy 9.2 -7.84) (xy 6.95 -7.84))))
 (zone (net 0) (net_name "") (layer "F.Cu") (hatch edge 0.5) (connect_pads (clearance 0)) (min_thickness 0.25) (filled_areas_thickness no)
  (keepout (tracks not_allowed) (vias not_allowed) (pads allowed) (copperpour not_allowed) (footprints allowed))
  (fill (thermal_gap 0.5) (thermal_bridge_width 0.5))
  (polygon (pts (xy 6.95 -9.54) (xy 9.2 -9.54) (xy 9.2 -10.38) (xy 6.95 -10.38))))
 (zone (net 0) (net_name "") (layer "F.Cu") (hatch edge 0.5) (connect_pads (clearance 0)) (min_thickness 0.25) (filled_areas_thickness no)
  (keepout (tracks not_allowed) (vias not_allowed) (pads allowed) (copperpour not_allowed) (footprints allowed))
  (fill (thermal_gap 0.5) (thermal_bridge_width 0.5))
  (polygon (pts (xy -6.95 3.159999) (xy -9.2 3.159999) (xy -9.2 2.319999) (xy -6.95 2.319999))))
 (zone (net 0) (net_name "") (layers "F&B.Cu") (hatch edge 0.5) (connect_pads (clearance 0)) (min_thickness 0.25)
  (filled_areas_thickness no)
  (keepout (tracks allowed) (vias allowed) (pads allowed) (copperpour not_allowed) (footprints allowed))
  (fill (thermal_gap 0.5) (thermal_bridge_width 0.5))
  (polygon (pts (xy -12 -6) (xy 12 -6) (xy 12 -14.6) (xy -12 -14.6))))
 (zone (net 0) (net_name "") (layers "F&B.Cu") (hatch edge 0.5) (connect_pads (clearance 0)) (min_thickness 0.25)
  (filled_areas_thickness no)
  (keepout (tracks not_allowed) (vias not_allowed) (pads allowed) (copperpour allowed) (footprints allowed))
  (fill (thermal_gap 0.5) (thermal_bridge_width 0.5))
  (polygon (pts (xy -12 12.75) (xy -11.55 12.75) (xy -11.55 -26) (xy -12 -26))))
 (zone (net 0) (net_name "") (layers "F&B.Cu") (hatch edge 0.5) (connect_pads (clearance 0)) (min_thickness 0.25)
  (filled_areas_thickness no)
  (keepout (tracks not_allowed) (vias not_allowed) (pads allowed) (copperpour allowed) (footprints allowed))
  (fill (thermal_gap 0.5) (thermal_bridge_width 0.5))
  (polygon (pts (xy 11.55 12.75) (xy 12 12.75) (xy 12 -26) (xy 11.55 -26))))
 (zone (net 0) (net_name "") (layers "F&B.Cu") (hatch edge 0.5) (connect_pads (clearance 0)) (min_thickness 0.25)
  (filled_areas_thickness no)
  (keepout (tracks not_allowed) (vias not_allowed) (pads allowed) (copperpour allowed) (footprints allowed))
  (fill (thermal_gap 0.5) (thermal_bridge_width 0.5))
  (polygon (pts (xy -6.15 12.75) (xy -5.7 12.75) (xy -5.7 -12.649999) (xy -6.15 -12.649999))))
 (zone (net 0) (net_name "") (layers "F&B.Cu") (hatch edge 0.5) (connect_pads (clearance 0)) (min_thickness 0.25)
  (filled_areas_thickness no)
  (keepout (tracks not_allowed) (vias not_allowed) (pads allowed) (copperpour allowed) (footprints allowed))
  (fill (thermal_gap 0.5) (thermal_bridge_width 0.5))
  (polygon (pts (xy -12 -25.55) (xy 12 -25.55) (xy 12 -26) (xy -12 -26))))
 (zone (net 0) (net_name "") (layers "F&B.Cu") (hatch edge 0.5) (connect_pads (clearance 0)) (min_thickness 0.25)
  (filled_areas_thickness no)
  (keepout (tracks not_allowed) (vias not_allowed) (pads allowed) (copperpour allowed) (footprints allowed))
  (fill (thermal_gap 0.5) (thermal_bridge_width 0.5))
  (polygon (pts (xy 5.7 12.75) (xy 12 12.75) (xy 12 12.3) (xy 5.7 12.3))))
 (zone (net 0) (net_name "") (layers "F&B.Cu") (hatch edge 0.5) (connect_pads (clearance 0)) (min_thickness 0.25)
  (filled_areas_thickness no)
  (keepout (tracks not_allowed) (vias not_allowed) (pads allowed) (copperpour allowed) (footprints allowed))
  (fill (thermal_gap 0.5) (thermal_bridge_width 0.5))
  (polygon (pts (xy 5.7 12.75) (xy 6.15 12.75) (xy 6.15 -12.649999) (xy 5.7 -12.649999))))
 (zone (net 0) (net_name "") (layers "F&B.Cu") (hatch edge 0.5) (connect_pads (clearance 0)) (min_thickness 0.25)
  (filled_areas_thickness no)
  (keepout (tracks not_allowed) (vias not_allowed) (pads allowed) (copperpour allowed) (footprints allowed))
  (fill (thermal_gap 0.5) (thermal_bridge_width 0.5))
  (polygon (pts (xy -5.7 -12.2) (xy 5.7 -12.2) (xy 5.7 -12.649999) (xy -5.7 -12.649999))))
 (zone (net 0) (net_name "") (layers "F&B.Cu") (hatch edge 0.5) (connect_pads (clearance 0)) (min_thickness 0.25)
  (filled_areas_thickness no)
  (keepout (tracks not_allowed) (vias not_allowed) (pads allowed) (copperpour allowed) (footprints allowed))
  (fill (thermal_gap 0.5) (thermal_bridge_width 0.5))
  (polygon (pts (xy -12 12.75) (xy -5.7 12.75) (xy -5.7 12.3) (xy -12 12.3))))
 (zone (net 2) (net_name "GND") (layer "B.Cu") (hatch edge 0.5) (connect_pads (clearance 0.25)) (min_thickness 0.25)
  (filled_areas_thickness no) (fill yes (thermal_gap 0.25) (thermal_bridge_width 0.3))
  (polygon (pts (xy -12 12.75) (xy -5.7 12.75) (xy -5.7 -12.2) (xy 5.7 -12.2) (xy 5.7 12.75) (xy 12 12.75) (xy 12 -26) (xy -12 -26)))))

